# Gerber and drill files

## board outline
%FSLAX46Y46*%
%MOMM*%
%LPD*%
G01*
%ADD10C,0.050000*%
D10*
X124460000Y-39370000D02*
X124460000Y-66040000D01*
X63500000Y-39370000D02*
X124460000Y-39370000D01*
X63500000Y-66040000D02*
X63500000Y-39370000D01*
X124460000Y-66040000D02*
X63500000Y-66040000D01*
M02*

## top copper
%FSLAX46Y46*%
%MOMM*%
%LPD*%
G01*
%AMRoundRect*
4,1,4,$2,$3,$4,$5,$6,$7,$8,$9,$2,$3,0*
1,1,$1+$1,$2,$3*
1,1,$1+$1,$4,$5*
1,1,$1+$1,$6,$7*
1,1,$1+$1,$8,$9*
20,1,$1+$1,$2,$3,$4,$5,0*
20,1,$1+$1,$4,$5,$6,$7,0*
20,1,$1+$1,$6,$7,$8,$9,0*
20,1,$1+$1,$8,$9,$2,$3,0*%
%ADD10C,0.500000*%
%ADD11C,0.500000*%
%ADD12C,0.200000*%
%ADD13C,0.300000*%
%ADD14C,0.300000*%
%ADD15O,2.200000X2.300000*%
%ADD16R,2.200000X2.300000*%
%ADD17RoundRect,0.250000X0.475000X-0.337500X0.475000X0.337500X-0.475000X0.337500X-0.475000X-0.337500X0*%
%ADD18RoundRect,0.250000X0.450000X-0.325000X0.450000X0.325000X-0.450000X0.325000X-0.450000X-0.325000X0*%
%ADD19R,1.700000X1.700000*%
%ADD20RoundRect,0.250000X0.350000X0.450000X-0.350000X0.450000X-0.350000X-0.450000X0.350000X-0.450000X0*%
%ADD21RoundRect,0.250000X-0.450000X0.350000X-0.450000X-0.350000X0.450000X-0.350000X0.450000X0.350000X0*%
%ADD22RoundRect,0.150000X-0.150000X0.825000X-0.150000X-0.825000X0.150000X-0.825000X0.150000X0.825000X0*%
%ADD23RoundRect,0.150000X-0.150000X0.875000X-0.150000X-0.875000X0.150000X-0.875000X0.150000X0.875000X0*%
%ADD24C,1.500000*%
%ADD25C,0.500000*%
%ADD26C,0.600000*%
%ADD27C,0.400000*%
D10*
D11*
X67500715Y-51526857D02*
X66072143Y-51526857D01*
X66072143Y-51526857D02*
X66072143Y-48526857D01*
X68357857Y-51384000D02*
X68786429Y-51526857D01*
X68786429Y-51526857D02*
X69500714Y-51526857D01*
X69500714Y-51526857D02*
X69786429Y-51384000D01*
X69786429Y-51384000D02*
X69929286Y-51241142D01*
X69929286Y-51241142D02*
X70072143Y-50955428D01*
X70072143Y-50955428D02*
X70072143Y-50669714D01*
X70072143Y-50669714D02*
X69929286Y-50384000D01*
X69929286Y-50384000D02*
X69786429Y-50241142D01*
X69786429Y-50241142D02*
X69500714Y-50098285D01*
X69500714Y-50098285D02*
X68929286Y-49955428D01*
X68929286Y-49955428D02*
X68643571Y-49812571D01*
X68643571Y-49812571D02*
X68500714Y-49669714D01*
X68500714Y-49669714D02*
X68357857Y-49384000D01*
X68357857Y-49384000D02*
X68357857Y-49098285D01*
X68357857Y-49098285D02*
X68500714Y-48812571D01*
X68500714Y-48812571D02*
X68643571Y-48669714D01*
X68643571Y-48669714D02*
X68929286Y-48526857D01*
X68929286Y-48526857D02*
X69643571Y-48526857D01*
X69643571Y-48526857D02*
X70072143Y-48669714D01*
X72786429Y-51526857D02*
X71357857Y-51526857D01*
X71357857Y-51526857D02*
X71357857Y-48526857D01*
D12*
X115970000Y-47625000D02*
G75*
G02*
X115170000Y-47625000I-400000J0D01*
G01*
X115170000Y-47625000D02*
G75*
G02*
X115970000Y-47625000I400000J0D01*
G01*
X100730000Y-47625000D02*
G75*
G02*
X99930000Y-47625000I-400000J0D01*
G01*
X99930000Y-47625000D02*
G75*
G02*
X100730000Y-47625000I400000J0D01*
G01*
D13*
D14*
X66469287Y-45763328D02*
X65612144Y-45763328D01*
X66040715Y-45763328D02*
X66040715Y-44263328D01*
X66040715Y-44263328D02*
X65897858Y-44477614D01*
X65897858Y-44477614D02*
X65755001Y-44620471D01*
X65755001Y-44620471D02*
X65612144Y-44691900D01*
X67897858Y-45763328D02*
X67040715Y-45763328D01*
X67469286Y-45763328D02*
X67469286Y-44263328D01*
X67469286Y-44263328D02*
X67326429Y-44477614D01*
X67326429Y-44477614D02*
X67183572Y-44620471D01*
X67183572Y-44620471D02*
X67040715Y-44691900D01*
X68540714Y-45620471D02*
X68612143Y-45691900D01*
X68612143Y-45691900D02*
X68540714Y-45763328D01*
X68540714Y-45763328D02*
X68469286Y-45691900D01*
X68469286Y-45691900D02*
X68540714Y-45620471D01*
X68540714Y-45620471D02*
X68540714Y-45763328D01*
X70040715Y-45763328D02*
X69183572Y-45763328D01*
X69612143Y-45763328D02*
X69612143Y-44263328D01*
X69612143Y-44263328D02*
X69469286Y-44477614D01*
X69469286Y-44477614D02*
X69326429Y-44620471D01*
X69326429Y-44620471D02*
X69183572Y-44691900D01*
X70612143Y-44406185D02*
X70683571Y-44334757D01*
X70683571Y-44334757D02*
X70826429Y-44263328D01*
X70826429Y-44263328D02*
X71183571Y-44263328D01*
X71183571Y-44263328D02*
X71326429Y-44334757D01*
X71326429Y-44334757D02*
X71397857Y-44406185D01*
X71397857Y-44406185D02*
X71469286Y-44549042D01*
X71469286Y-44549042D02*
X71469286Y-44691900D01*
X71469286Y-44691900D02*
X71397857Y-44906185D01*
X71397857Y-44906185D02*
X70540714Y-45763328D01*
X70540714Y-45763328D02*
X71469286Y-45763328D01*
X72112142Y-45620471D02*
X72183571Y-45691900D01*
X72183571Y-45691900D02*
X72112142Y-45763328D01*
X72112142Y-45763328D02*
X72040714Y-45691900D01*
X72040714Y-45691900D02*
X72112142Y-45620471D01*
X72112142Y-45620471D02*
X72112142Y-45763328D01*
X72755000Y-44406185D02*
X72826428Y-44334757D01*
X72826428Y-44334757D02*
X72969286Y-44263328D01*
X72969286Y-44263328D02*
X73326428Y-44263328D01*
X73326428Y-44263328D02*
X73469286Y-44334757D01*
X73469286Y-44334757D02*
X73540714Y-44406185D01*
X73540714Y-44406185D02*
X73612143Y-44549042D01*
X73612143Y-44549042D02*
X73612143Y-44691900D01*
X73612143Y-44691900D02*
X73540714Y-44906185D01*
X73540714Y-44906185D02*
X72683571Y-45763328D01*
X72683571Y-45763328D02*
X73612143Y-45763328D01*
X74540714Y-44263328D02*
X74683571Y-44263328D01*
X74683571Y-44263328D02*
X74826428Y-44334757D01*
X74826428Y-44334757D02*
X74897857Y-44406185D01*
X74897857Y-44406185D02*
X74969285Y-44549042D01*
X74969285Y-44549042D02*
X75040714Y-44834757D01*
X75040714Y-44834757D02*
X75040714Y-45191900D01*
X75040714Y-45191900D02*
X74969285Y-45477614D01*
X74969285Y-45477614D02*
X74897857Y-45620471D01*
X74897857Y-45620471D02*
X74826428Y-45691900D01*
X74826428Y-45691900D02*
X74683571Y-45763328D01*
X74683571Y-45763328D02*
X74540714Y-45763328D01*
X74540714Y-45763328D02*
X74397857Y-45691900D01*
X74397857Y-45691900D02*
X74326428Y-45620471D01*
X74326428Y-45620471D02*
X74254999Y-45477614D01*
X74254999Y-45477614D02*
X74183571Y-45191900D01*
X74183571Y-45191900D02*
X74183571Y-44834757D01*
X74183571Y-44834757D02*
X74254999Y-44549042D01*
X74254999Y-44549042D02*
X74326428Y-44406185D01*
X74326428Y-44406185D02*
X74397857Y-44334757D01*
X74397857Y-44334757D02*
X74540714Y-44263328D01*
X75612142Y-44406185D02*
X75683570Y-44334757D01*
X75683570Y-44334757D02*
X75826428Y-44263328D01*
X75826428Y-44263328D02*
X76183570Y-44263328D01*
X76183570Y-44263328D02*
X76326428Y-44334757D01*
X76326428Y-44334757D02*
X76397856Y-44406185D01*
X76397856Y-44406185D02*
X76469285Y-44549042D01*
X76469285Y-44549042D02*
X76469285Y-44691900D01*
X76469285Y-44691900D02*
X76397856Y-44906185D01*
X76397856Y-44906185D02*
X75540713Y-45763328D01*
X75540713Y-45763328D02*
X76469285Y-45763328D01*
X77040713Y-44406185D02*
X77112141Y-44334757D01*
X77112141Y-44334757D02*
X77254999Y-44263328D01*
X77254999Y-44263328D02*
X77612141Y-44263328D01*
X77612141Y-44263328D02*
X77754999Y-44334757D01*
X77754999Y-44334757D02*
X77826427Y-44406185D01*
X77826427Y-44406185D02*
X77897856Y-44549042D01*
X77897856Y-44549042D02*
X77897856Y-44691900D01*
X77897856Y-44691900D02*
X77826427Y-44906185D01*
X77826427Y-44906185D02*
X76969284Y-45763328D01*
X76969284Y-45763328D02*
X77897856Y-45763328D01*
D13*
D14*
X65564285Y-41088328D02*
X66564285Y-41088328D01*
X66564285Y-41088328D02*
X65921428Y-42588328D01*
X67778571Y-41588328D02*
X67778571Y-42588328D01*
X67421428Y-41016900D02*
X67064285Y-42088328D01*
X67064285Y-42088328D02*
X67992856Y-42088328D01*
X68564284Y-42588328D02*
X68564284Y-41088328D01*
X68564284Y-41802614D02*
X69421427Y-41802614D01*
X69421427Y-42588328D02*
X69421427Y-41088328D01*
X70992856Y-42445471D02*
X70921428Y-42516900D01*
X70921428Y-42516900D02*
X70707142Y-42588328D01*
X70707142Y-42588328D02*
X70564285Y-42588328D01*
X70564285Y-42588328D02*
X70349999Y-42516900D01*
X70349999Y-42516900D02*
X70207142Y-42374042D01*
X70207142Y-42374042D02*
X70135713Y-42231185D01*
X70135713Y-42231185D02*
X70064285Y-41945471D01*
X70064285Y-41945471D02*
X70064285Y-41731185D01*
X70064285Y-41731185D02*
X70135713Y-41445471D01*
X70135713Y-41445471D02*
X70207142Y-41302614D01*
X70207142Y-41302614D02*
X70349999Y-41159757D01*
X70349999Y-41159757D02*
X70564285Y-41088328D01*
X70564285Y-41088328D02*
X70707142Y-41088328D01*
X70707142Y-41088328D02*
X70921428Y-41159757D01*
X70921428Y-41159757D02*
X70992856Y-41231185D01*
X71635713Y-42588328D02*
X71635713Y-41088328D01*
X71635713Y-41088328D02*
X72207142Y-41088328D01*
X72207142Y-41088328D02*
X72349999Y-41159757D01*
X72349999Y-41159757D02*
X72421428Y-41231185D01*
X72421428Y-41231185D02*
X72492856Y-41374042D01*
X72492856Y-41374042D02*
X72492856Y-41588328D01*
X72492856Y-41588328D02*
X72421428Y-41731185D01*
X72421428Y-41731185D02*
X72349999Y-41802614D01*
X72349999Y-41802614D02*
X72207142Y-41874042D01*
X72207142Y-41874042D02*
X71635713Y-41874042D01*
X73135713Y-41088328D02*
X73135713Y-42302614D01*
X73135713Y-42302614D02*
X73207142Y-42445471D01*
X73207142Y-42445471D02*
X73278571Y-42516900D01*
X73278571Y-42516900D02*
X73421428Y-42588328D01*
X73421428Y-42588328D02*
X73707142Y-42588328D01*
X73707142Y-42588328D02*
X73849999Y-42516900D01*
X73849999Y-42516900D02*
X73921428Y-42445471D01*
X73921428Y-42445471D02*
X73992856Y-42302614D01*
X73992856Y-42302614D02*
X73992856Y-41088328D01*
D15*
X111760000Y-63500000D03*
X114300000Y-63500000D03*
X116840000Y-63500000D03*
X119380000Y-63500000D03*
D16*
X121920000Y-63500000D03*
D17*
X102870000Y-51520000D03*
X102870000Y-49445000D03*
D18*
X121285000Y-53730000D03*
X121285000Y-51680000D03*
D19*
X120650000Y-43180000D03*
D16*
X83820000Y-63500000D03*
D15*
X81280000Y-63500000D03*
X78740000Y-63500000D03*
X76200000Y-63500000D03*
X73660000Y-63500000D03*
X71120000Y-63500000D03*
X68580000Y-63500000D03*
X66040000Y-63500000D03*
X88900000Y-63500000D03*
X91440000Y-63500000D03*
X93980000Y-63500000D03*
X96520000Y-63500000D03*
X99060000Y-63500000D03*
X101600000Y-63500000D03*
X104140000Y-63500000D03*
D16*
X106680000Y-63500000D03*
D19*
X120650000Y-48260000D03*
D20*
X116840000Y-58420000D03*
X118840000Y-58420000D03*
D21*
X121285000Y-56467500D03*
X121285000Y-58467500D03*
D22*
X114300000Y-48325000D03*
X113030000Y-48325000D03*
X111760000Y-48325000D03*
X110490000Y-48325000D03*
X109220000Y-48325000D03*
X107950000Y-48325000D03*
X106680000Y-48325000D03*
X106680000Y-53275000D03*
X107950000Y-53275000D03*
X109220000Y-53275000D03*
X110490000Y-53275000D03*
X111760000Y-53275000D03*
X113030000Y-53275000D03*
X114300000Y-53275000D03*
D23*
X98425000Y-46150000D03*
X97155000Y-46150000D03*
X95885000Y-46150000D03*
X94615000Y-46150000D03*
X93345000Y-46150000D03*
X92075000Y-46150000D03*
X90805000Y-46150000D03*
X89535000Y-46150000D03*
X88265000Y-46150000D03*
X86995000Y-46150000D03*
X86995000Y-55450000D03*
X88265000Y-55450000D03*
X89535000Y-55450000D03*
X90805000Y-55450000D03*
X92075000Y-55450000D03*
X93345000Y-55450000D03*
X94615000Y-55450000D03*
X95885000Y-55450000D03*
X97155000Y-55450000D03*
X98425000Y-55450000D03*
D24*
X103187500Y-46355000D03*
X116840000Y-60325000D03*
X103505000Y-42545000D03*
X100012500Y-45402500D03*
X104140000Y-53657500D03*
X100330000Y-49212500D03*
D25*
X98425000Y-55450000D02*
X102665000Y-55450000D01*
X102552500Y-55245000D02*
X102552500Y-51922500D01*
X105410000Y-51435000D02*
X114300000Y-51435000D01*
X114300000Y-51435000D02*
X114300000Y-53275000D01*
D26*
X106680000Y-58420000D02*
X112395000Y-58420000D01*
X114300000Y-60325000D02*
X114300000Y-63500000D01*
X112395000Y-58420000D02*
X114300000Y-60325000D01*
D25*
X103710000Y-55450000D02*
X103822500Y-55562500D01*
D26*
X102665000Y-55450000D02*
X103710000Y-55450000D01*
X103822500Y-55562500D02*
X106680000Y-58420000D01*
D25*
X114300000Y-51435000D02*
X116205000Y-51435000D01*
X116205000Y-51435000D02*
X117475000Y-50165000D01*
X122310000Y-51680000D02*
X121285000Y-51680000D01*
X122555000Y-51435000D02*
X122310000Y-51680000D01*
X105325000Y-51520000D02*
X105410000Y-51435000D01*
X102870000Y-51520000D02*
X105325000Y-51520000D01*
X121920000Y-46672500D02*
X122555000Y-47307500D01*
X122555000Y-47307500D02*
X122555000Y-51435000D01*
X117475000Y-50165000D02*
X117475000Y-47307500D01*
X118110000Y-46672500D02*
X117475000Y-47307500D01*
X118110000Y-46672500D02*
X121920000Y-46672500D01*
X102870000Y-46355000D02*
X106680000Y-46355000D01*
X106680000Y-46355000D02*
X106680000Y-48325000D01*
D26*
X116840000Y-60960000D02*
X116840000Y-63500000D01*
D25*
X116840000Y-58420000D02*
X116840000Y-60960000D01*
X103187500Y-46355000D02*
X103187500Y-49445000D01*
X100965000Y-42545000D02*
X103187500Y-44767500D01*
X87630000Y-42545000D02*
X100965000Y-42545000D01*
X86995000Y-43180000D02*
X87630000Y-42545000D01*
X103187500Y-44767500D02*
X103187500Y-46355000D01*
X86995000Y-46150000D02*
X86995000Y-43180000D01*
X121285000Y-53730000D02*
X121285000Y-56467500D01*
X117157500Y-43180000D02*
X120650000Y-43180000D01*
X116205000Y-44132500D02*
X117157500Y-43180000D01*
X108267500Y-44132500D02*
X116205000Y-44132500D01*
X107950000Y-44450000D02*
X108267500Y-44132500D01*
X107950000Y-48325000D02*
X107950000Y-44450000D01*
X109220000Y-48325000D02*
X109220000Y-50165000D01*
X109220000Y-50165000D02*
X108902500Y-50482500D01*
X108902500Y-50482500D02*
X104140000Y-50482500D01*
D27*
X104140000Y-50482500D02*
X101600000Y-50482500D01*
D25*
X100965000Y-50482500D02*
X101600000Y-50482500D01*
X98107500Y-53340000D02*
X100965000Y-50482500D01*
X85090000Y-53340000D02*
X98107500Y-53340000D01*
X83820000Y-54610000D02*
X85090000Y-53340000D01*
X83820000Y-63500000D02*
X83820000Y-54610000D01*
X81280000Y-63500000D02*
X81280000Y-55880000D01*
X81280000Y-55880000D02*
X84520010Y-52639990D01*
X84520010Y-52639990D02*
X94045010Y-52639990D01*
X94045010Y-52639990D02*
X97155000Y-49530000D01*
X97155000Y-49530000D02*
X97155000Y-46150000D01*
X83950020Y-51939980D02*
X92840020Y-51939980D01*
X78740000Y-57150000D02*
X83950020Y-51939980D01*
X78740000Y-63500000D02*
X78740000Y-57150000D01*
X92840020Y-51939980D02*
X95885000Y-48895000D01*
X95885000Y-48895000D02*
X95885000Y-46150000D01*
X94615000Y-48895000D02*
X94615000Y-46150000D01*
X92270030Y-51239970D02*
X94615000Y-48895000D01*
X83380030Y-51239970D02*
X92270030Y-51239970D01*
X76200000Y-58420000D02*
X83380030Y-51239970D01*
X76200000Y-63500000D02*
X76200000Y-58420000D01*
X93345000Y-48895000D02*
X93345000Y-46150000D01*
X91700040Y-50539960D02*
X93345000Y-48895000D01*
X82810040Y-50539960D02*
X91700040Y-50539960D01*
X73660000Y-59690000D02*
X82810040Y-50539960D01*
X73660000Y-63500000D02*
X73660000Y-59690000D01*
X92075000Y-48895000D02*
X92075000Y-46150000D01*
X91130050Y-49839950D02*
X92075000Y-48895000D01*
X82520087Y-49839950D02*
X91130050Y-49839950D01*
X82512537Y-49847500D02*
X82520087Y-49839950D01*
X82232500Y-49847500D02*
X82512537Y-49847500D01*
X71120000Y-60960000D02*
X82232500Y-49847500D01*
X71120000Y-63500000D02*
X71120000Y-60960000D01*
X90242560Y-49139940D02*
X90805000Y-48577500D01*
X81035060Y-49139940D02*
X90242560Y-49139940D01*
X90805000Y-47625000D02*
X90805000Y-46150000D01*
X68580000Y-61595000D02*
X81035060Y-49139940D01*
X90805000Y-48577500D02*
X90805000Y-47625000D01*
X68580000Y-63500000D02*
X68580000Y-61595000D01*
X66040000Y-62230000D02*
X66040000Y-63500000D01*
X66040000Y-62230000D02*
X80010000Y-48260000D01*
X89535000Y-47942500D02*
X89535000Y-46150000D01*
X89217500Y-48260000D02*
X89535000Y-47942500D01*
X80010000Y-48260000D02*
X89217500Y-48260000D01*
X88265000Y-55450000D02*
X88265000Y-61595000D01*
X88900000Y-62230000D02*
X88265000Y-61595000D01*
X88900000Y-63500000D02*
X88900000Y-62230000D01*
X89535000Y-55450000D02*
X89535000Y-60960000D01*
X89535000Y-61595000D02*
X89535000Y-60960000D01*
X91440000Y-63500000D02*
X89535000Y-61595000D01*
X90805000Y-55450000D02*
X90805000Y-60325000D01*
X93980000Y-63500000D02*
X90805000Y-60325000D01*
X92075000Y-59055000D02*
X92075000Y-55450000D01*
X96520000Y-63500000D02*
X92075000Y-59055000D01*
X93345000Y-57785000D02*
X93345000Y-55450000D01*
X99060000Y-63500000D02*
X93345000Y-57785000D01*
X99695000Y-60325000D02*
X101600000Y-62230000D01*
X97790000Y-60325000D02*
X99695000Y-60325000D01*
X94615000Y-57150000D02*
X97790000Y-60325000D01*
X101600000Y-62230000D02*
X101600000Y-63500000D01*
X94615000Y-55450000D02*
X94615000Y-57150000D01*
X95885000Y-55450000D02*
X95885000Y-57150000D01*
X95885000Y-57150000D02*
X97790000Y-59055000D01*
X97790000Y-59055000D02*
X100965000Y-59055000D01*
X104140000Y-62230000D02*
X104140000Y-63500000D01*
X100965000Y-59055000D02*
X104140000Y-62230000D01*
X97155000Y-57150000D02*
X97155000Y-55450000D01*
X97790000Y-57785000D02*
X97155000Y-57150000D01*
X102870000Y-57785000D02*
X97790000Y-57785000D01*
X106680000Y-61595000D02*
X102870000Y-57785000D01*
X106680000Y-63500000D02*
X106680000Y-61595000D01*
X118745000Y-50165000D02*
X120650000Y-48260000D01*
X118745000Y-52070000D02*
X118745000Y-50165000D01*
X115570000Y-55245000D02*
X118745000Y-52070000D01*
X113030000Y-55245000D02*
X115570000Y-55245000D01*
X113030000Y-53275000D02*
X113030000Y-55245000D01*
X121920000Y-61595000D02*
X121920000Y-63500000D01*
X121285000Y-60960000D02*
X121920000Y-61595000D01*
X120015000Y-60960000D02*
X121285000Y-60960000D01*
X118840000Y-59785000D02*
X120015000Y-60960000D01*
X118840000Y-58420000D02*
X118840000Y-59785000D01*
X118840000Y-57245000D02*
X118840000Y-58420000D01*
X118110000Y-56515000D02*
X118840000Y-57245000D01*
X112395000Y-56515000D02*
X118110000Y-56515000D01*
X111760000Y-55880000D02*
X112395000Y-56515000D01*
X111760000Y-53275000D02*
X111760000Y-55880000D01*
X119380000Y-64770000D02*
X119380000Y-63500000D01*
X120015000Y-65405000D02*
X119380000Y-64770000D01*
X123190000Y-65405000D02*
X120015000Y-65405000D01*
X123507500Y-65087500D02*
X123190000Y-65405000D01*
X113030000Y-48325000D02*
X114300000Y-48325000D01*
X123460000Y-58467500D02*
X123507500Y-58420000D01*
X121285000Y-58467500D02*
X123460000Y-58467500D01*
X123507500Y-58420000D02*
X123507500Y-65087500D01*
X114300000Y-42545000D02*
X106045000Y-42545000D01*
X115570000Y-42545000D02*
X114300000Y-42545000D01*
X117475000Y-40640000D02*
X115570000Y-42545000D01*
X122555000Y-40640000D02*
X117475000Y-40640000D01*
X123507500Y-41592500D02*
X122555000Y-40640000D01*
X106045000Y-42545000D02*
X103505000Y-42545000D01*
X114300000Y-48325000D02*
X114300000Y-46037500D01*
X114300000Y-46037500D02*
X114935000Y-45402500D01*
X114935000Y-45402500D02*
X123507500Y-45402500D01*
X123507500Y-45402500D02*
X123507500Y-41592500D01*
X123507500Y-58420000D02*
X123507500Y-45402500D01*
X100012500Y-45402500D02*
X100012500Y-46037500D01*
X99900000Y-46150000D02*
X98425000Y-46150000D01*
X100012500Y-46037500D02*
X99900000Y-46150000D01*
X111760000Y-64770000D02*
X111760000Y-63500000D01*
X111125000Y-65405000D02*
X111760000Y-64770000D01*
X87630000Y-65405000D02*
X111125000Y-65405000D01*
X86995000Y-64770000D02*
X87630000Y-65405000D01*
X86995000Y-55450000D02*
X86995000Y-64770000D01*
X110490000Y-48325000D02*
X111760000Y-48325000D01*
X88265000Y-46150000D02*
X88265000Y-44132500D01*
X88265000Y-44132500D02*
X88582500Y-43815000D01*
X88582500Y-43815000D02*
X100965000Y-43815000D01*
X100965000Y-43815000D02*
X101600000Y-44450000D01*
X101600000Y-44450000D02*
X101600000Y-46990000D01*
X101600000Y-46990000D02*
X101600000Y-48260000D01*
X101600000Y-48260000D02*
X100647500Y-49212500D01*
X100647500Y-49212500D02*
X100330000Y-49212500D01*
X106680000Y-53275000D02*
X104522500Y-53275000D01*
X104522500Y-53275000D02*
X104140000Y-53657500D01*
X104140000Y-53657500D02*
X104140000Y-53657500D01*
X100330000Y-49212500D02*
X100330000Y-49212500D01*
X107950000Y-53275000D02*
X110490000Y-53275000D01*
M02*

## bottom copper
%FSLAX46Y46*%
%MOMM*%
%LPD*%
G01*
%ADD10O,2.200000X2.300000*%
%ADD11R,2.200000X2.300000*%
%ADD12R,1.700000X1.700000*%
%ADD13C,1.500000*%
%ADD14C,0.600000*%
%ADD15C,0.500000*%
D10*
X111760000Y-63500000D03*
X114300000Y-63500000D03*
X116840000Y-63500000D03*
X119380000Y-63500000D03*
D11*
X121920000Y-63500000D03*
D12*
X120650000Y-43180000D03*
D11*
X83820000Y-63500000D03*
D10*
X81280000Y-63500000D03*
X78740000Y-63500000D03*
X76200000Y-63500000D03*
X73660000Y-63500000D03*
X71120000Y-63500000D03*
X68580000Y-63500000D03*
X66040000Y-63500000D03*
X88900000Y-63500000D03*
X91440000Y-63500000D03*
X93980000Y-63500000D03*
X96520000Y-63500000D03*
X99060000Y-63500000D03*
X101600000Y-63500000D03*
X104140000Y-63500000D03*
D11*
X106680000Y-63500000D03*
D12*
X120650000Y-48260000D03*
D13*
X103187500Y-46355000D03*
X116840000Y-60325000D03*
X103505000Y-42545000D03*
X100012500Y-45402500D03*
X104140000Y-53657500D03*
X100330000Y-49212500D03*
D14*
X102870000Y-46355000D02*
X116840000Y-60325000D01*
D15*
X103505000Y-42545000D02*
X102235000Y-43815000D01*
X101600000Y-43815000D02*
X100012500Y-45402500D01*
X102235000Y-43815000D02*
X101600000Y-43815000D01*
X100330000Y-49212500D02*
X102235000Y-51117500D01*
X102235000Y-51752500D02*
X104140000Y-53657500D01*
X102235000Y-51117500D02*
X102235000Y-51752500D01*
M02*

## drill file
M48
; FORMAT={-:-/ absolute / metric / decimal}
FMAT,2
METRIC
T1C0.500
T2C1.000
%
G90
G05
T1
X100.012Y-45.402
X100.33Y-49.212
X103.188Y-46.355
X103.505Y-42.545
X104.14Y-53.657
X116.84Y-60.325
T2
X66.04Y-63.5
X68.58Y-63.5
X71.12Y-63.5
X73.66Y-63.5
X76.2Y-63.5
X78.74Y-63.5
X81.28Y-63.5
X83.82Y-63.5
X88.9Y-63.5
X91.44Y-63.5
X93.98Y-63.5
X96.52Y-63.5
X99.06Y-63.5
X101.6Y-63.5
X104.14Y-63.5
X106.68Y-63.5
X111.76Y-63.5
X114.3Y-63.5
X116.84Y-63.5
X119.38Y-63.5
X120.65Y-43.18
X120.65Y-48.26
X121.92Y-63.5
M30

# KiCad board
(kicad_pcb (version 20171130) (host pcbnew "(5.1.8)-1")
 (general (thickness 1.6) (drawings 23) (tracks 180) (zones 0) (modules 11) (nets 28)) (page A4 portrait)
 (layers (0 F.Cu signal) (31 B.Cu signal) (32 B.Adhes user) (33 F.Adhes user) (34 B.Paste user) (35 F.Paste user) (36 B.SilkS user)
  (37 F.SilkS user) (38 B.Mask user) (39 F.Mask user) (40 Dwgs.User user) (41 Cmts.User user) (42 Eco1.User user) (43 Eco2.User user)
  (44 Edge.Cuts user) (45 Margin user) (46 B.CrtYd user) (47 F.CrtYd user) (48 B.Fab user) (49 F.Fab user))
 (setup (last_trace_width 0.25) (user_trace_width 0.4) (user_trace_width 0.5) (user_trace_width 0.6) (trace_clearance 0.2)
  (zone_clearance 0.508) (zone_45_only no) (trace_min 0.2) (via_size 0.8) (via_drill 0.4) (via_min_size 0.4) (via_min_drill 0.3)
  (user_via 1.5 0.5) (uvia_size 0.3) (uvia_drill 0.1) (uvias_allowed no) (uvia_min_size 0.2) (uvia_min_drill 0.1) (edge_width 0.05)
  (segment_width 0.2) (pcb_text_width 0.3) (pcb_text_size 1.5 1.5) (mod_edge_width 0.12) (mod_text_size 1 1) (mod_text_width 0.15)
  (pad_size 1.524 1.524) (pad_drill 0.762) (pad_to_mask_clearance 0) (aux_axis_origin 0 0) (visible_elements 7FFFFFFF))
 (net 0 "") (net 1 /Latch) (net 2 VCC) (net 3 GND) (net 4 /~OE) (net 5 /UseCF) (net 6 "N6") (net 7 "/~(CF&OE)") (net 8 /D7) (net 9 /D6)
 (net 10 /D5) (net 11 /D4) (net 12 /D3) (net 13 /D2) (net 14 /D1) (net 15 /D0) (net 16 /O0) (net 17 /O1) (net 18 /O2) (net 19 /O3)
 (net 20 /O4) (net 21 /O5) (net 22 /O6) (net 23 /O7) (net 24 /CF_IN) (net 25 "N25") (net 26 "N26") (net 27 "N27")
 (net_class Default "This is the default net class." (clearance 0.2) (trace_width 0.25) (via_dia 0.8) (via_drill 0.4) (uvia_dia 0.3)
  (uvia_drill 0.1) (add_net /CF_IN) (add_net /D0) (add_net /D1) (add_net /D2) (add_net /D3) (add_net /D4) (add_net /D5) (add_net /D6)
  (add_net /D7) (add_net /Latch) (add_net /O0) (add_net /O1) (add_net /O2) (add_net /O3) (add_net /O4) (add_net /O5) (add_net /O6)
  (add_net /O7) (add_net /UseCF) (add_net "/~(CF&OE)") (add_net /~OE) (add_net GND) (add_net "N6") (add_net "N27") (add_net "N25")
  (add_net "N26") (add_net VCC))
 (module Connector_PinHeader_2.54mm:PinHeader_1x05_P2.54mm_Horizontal (layer F.Cu) (at 121.92 63.5 270)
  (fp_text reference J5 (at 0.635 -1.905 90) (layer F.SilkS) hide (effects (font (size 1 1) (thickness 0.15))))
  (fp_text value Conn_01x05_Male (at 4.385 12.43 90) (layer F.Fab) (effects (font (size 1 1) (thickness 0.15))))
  (pad 5 thru_hole oval (at 0 10.16 270) (size 2.3 2.2) (drill 1) (layers *.Cu *.Mask) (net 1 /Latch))
  (pad 4 thru_hole oval (at 0 7.62 270) (size 2.3 2.2) (drill 1) (layers *.Cu *.Mask) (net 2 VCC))
  (pad 3 thru_hole oval (at 0 5.08 270) (size 2.3 2.2) (drill 1) (layers *.Cu *.Mask) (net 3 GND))
  (pad 2 thru_hole oval (at 0 2.54 270) (size 2.3 2.2) (drill 1) (layers *.Cu *.Mask) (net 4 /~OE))
  (pad 1 thru_hole rect (at 0 0 270) (size 2.3 2.2) (drill 1) (layers *.Cu *.Mask) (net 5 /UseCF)))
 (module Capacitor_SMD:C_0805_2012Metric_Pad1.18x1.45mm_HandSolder (layer F.Cu) (at 102.87 50.4825 90)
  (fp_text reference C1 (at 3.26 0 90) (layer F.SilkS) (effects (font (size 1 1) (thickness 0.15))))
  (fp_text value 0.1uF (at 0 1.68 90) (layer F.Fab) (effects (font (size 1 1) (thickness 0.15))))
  (pad 1 smd roundrect (at -1.0375 0 90) (size 1.175 1.45) (layers F.Cu F.Paste F.Mask) (roundrect_rratio 0.212766) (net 2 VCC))
  (pad 2 smd roundrect (at 1.0375 0 90) (size 1.175 1.45) (layers F.Cu F.Paste F.Mask) (roundrect_rratio 0.212766) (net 3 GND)))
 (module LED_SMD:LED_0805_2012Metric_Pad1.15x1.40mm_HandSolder (layer F.Cu) (at 121.285 52.705 90)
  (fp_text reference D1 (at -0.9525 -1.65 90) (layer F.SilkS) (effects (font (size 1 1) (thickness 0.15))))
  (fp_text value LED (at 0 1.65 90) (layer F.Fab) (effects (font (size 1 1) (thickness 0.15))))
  (pad 1 smd roundrect (at -1.025 0 90) (size 1.15 1.4) (layers F.Cu F.Paste F.Mask) (roundrect_rratio 0.217391) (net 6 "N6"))
  (pad 2 smd roundrect (at 1.025 0 90) (size 1.15 1.4) (layers F.Cu F.Paste F.Mask) (roundrect_rratio 0.217391) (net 2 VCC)))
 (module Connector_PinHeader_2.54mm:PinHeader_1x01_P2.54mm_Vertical (layer F.Cu) (at 120.65 43.18)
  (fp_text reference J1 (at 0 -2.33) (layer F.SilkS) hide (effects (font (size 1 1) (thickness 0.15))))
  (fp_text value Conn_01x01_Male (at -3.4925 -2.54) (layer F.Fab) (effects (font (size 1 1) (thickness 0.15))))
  (pad 1 thru_hole rect (at 0 0) (size 1.7 1.7) (drill 1) (layers *.Cu *.Mask) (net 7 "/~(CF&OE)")))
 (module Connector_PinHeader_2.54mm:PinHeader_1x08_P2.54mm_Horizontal (layer F.Cu) (at 83.82 63.5 270)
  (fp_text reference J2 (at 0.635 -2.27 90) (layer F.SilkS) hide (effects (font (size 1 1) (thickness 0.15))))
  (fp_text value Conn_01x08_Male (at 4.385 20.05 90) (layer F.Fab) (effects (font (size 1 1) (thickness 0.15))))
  (pad 1 thru_hole rect (at 0 0 270) (size 2.3 2.2) (drill 1) (layers *.Cu *.Mask) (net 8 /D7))
  (pad 2 thru_hole oval (at 0 2.54 270) (size 2.3 2.2) (drill 1) (layers *.Cu *.Mask) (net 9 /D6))
  (pad 3 thru_hole oval (at 0 5.08 270) (size 2.3 2.2) (drill 1) (layers *.Cu *.Mask) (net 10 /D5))
  (pad 4 thru_hole oval (at 0 7.62 270) (size 2.3 2.2) (drill 1) (layers *.Cu *.Mask) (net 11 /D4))
  (pad 5 thru_hole oval (at 0 10.16 270) (size 2.3 2.2) (drill 1) (layers *.Cu *.Mask) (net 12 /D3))
  (pad 6 thru_hole oval (at 0 12.7 270) (size 2.3 2.2) (drill 1) (layers *.Cu *.Mask) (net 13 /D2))
  (pad 7 thru_hole oval (at 0 15.24 270) (size 2.3 2.2) (drill 1) (layers *.Cu *.Mask) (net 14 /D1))
  (pad 8 thru_hole oval (at 0 17.78 270) (size 2.3 2.2) (drill 1) (layers *.Cu *.Mask) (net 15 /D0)))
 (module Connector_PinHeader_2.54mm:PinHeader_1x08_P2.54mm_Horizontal (layer F.Cu) (at 106.68 63.5 270)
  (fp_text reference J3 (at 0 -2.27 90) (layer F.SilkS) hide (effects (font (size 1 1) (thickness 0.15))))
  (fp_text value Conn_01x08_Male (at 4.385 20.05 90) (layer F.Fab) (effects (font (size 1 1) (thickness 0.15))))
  (pad 8 thru_hole oval (at 0 17.78 270) (size 2.3 2.2) (drill 1) (layers *.Cu *.Mask) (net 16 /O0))
  (pad 7 thru_hole oval (at 0 15.24 270) (size 2.3 2.2) (drill 1) (layers *.Cu *.Mask) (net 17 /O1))
  (pad 6 thru_hole oval (at 0 12.7 270) (size 2.3 2.2) (drill 1) (layers *.Cu *.Mask) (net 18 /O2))
  (pad 5 thru_hole oval (at 0 10.16 270) (size 2.3 2.2) (drill 1) (layers *.Cu *.Mask) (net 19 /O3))
  (pad 4 thru_hole oval (at 0 7.62 270) (size 2.3 2.2) (drill 1) (layers *.Cu *.Mask) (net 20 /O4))
  (pad 3 thru_hole oval (at 0 5.08 270) (size 2.3 2.2) (drill 1) (layers *.Cu *.Mask) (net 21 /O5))
  (pad 2 thru_hole oval (at 0 2.54 270) (size 2.3 2.2) (drill 1) (layers *.Cu *.Mask) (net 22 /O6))
  (pad 1 thru_hole rect (at 0 0 270) (size 2.3 2.2) (drill 1) (layers *.Cu *.Mask) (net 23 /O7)))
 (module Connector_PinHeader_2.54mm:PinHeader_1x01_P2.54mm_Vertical (layer F.Cu) (at 120.65 48.26)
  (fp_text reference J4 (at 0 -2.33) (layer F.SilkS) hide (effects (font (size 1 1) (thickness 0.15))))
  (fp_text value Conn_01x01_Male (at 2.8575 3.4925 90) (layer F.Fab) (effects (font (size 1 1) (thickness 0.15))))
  (pad 1 thru_hole rect (at 0 0) (size 1.7 1.7) (drill 1) (layers *.Cu *.Mask) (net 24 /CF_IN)))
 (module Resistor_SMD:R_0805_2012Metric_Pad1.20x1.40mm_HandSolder (layer F.Cu) (at 117.84 58.42 180)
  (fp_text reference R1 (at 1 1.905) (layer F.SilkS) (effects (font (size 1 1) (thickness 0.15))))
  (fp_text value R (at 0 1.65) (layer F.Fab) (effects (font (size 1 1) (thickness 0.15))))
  (pad 2 smd roundrect (at 1 0 180) (size 1.2 1.4) (layers F.Cu F.Paste F.Mask) (roundrect_rratio 0.208333) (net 3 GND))
  (pad 1 smd roundrect (at -1 0 180) (size 1.2 1.4) (layers F.Cu F.Paste F.Mask) (roundrect_rratio 0.208333) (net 5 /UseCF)))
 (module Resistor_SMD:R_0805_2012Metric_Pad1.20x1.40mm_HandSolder (layer F.Cu) (at 121.285 57.4675 270)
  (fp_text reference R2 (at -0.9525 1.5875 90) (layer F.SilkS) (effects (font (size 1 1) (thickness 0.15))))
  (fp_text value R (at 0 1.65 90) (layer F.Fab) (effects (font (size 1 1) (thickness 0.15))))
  (pad 1 smd roundrect (at -1 0 270) (size 1.2 1.4) (layers F.Cu F.Paste F.Mask) (roundrect_rratio 0.208333) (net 6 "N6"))
  (pad 2 smd roundrect (at 1 0 270) (size 1.2 1.4) (layers F.Cu F.Paste F.Mask) (roundrect_rratio 0.208333) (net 4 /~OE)))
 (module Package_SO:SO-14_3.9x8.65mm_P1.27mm (layer F.Cu) (at 110.49 50.8 270)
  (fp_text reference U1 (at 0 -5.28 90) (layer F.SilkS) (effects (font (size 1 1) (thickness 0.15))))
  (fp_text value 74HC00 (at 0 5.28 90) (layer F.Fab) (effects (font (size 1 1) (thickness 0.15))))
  (pad 1 smd roundrect (at -2.475 -3.81 270) (size 1.95 0.6) (layers F.Cu F.Paste F.Mask) (roundrect_rratio 0.25) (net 4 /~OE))
  (pad 2 smd roundrect (at -2.475 -2.54 270) (size 1.95 0.6) (layers F.Cu F.Paste F.Mask) (roundrect_rratio 0.25) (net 4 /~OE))
  (pad 3 smd roundrect (at -2.475 -1.27 270) (size 1.95 0.6) (layers F.Cu F.Paste F.Mask) (roundrect_rratio 0.25) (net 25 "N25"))
  (pad 4 smd roundrect (at -2.475 0 270) (size 1.95 0.6) (layers F.Cu F.Paste F.Mask) (roundrect_rratio 0.25) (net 25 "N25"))
  (pad 5 smd roundrect (at -2.475 1.27 270) (size 1.95 0.6) (layers F.Cu F.Paste F.Mask) (roundrect_rratio 0.25) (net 8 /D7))
  (pad 6 smd roundrect (at -2.475 2.54 270) (size 1.95 0.6) (layers F.Cu F.Paste F.Mask) (roundrect_rratio 0.25) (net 7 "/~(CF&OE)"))
  (pad 7 smd roundrect (at -2.475 3.81 270) (size 1.95 0.6) (layers F.Cu F.Paste F.Mask) (roundrect_rratio 0.25) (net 3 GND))
  (pad 8 smd roundrect (at 2.475 3.81 270) (size 1.95 0.6) (layers F.Cu F.Paste F.Mask) (roundrect_rratio 0.25) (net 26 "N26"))
  (pad 9 smd roundrect (at 2.475 2.54 270) (size 1.95 0.6) (layers F.Cu F.Paste F.Mask) (roundrect_rratio 0.25) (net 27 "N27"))
  (pad 10 smd roundrect (at 2.475 1.27 270) (size 1.95 0.6) (layers F.Cu F.Paste F.Mask) (roundrect_rratio 0.25) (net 27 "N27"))
  (pad 11 smd roundrect (at 2.475 0 270) (size 1.95 0.6) (layers F.Cu F.Paste F.Mask) (roundrect_rratio 0.25) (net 27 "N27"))
  (pad 12 smd roundrect (at 2.475 -1.27 270) (size 1.95 0.6) (layers F.Cu F.Paste F.Mask) (roundrect_rratio 0.25) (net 5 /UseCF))
  (pad 13 smd roundrect (at 2.475 -2.54 270) (size 1.95 0.6) (layers F.Cu F.Paste F.Mask) (roundrect_rratio 0.25) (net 24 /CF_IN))
  (pad 14 smd roundrect (at 2.475 -3.81 270) (size 1.95 0.6) (layers F.Cu F.Paste F.Mask) (roundrect_rratio 0.25) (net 2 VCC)))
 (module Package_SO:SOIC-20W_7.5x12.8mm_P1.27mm (layer F.Cu) (at 92.71 50.8 270)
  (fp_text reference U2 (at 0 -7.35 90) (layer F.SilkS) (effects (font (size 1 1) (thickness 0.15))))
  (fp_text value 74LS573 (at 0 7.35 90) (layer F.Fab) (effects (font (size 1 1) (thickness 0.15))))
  (pad 1 smd roundrect (at -4.65 -5.715 270) (size 2.05 0.6) (layers F.Cu F.Paste F.Mask) (roundrect_rratio 0.25) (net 4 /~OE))
  (pad 2 smd roundrect (at -4.65 -4.445 270) (size 2.05 0.6) (layers F.Cu F.Paste F.Mask) (roundrect_rratio 0.25) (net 9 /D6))
  (pad 3 smd roundrect (at -4.65 -3.175 270) (size 2.05 0.6) (layers F.Cu F.Paste F.Mask) (roundrect_rratio 0.25) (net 10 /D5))
  (pad 4 smd roundrect (at -4.65 -1.905 270) (size 2.05 0.6) (layers F.Cu F.Paste F.Mask) (roundrect_rratio 0.25) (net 11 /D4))
  (pad 5 smd roundrect (at -4.65 -0.635 270) (size 2.05 0.6) (layers F.Cu F.Paste F.Mask) (roundrect_rratio 0.25) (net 12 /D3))
  (pad 6 smd roundrect (at -4.65 0.635 270) (size 2.05 0.6) (layers F.Cu F.Paste F.Mask) (roundrect_rratio 0.25) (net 13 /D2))
  (pad 7 smd roundrect (at -4.65 1.905 270) (size 2.05 0.6) (layers F.Cu F.Paste F.Mask) (roundrect_rratio 0.25) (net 14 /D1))
  (pad 8 smd roundrect (at -4.65 3.175 270) (size 2.05 0.6) (layers F.Cu F.Paste F.Mask) (roundrect_rratio 0.25) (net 15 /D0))
  (pad 9 smd roundrect (at -4.65 4.445 270) (size 2.05 0.6) (layers F.Cu F.Paste F.Mask) (roundrect_rratio 0.25) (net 26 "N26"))
  (pad 10 smd roundrect (at -4.65 5.715 270) (size 2.05 0.6) (layers F.Cu F.Paste F.Mask) (roundrect_rratio 0.25) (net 3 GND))
  (pad 11 smd roundrect (at 4.65 5.715 270) (size 2.05 0.6) (layers F.Cu F.Paste F.Mask) (roundrect_rratio 0.25) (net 1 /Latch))
  (pad 12 smd roundrect (at 4.65 4.445 270) (size 2.05 0.6) (layers F.Cu F.Paste F.Mask) (roundrect_rratio 0.25) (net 16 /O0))
  (pad 13 smd roundrect (at 4.65 3.175 270) (size 2.05 0.6) (layers F.Cu F.Paste F.Mask) (roundrect_rratio 0.25) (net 17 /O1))
  (pad 14 smd roundrect (at 4.65 1.905 270) (size 2.05 0.6) (layers F.Cu F.Paste F.Mask) (roundrect_rratio 0.25) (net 18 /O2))
  (pad 15 smd roundrect (at 4.65 0.635 270) (size 2.05 0.6) (layers F.Cu F.Paste F.Mask) (roundrect_rratio 0.25) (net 19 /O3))
  (pad 16 smd roundrect (at 4.65 -0.635 270) (size 2.05 0.6) (layers F.Cu F.Paste F.Mask) (roundrect_rratio 0.25) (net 20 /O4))
  (pad 17 smd roundrect (at 4.65 -1.905 270) (size 2.05 0.6) (layers F.Cu F.Paste F.Mask) (roundrect_rratio 0.25) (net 21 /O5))
  (pad 18 smd roundrect (at 4.65 -3.175 270) (size 2.05 0.6) (layers F.Cu F.Paste F.Mask) (roundrect_rratio 0.25) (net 22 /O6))
  (pad 19 smd roundrect (at 4.65 -4.445 270) (size 2.05 0.6) (layers F.Cu F.Paste F.Mask) (roundrect_rratio 0.25) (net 23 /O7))
  (pad 20 smd roundrect (at 4.65 -5.715 270) (size 2.05 0.6) (layers F.Cu F.Paste F.Mask) (roundrect_rratio 0.25) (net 2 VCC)))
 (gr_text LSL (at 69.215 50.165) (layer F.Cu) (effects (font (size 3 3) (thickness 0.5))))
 (gr_circle (center 115.57 47.625) (end 115.97 47.625) (layer F.Cu) (width 0.2))
 (gr_circle (center 100.33 47.625) (end 100.73 47.625) (layer F.Cu) (width 0.2))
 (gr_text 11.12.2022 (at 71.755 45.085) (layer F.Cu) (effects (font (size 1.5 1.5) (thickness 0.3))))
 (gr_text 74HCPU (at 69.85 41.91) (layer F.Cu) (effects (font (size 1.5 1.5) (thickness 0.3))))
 (gr_line (start 124.46 39.37) (end 124.46 66.04) (layer Edge.Cuts) (width 0.05))
 (gr_line (start 63.5 39.37) (end 124.46 39.37) (layer Edge.Cuts) (width 0.05))
 (gr_line (start 63.5 66.04) (end 63.5 39.37) (layer Edge.Cuts) (width 0.05))
 (gr_line (start 124.46 66.04) (end 63.5 66.04) (layer Edge.Cuts) (width 0.05))
 (segment (start 98.425 55.45) (end 102.665 55.45) (width 0.5) (layer F.Cu) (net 2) (status 10))
 (segment (start 102.5525 55.245) (end 102.5525 51.9225) (width 0.5) (layer F.Cu) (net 2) (status 20))
 (segment (start 105.41 51.435) (end 114.3 51.435) (width 0.5) (layer F.Cu) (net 2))
 (segment (start 114.3 51.435) (end 114.3 53.275) (width 0.5) (layer F.Cu) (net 2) (status 20))
 (segment (start 106.68 58.42) (end 112.395 58.42) (width 0.6) (layer F.Cu) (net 2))
 (segment (start 114.3 60.325) (end 114.3 63.5) (width 0.6) (layer F.Cu) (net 2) (status 20))
 (segment (start 112.395 58.42) (end 114.3 60.325) (width 0.6) (layer F.Cu) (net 2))
 (segment (start 103.71 55.45) (end 103.8225 55.5625) (width 0.5) (layer F.Cu) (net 2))
 (segment (start 102.665 55.45) (end 103.71 55.45) (width 0.6) (layer F.Cu) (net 2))
 (segment (start 103.8225 55.5625) (end 106.68 58.42) (width 0.6) (layer F.Cu) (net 2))
 (segment (start 114.3 51.435) (end 116.205 51.435) (width 0.5) (layer F.Cu) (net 2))
 (segment (start 116.205 51.435) (end 117.475 50.165) (width 0.5) (layer F.Cu) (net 2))
 (segment (start 122.31 51.68) (end 121.285 51.68) (width 0.5) (layer F.Cu) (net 2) (status 20))
 (segment (start 122.555 51.435) (end 122.31 51.68) (width 0.5) (layer F.Cu) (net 2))
 (segment (start 105.325 51.52) (end 105.41 51.435) (width 0.5) (layer F.Cu) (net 2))
 (segment (start 102.87 51.52) (end 105.325 51.52) (width 0.5) (layer F.Cu) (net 2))
 (segment (start 121.92 46.6725) (end 122.555 47.3075) (width 0.5) (layer F.Cu) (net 2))
 (segment (start 122.555 47.3075) (end 122.555 51.435) (width 0.5) (layer F.Cu) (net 2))
 (segment (start 117.475 50.165) (end 117.475 47.3075) (width 0.5) (layer F.Cu) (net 2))
 (segment (start 118.11 46.6725) (end 117.475 47.3075) (width 0.5) (layer F.Cu) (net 2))
 (segment (start 118.11 46.6725) (end 121.92 46.6725) (width 0.5) (layer F.Cu) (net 2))
 (segment (start 102.87 46.355) (end 106.68 46.355) (width 0.5) (layer F.Cu) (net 3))
 (segment (start 106.68 46.355) (end 106.68 48.325) (width 0.5) (layer F.Cu) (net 3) (status 20))
 (segment (start 116.84 60.96) (end 116.84 63.5) (width 0.6) (layer F.Cu) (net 3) (status 20))
 (segment (start 116.84 58.42) (end 116.84 60.96) (width 0.5) (layer F.Cu) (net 3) (status 10))
 (segment (start 103.1875 46.355) (end 103.1875 49.445) (width 0.5) (layer F.Cu) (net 3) (status 20))
 (via (at 103.1875 46.355) (size 1.5) (drill 0.5) (layers F.Cu B.Cu) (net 3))
 (segment (start 102.87 46.355) (end 116.84 60.325) (width 0.6) (layer B.Cu) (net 3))
 (via (at 116.84 60.325) (size 1.5) (drill 0.5) (layers F.Cu B.Cu) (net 3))
 (segment (start 100.965 42.545) (end 103.1875 44.7675) (width 0.5) (layer F.Cu) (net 3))
 (segment (start 87.63 42.545) (end 100.965 42.545) (width 0.5) (layer F.Cu) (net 3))
 (segment (start 86.995 43.18) (end 87.63 42.545) (width 0.5) (layer F.Cu) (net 3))
 (segment (start 103.1875 44.7675) (end 103.1875 46.355) (width 0.5) (layer F.Cu) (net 3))
 (segment (start 86.995 46.15) (end 86.995 43.18) (width 0.5) (layer F.Cu) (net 3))
 (segment (start 121.285 53.73) (end 121.285 56.4675) (width 0.5) (layer F.Cu) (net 6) (status 30))
 (segment (start 117.1575 43.18) (end 120.65 43.18) (width 0.5) (layer F.Cu) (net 7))
 (segment (start 116.205 44.1325) (end 117.1575 43.18) (width 0.5) (layer F.Cu) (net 7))
 (segment (start 108.2675 44.1325) (end 116.205 44.1325) (width 0.5) (layer F.Cu) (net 7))
 (segment (start 107.95 44.45) (end 108.2675 44.1325) (width 0.5) (layer F.Cu) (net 7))
 (segment (start 107.95 48.325) (end 107.95 44.45) (width 0.5) (layer F.Cu) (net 7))
 (segment (start 109.22 48.325) (end 109.22 50.165) (width 0.5) (layer F.Cu) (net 8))
 (segment (start 109.22 50.165) (end 108.9025 50.4825) (width 0.5) (layer F.Cu) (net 8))
 (segment (start 108.9025 50.4825) (end 104.14 50.4825) (width 0.5) (layer F.Cu) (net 8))
 (segment (start 104.14 50.4825) (end 101.6 50.4825) (width 0.4) (layer F.Cu) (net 8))
 (segment (start 100.965 50.4825) (end 101.6 50.4825) (width 0.5) (layer F.Cu) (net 8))
 (segment (start 98.1075 53.34) (end 100.965 50.4825) (width 0.5) (layer F.Cu) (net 8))
 (segment (start 85.09 53.34) (end 98.1075 53.34) (width 0.5) (layer F.Cu) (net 8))
 (segment (start 83.82 54.61) (end 85.09 53.34) (width 0.5) (layer F.Cu) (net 8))
 (segment (start 83.82 63.5) (end 83.82 54.61) (width 0.5) (layer F.Cu) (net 8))
 (segment (start 81.28 63.5) (end 81.28 55.88) (width 0.5) (layer F.Cu) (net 9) (status 10))
 (segment (start 81.28 55.88) (end 84.52001 52.63999) (width 0.5) (layer F.Cu) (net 9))
 (segment (start 84.52001 52.63999) (end 94.04501 52.63999) (width 0.5) (layer F.Cu) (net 9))
 (segment (start 94.04501 52.63999) (end 97.155 49.53) (width 0.5) (layer F.Cu) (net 9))
 (segment (start 97.155 49.53) (end 97.155 46.15) (width 0.5) (layer F.Cu) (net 9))
 (segment (start 83.95002 51.93998) (end 92.84002 51.93998) (width 0.5) (layer F.Cu) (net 10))
 (segment (start 78.74 57.15) (end 83.95002 51.93998) (width 0.5) (layer F.Cu) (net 10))
 (segment (start 78.74 63.5) (end 78.74 57.15) (width 0.5) (layer F.Cu) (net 10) (status 10))
 (segment (start 92.84002 51.93998) (end 95.885 48.895) (width 0.5) (layer F.Cu) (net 10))
 (segment (start 95.885 48.895) (end 95.885 46.15) (width 0.5) (layer F.Cu) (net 10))
 (segment (start 94.615 48.895) (end 94.615 46.15) (width 0.5) (layer F.Cu) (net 11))
 (segment (start 92.27003 51.23997) (end 94.615 48.895) (width 0.5) (layer F.Cu) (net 11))
 (segment (start 83.38003 51.23997) (end 92.27003 51.23997) (width 0.5) (layer F.Cu) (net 11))
 (segment (start 76.2 58.42) (end 83.38003 51.23997) (width 0.5) (layer F.Cu) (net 11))
 (segment (start 76.2 63.5) (end 76.2 58.42) (width 0.5) (layer F.Cu) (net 11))
 (segment (start 93.345 48.895) (end 93.345 46.15) (width 0.5) (layer F.Cu) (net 12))
 (segment (start 91.70004 50.53996) (end 93.345 48.895) (width 0.5) (layer F.Cu) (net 12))
 (segment (start 82.81004 50.53996) (end 91.70004 50.53996) (width 0.5) (layer F.Cu) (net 12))
 (segment (start 73.66 59.69) (end 82.81004 50.53996) (width 0.5) (layer F.Cu) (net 12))
 (segment (start 73.66 63.5) (end 73.66 59.69) (width 0.5) (layer F.Cu) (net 12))
 (segment (start 92.075 48.895) (end 92.075 46.15) (width 0.5) (layer F.Cu) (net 13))
 (segment (start 91.13005 49.83995) (end 92.075 48.895) (width 0.5) (layer F.Cu) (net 13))
 (segment (start 82.520087 49.83995) (end 91.13005 49.83995) (width 0.5) (layer F.Cu) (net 13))
 (segment (start 82.512537 49.8475) (end 82.520087 49.83995) (width 0.5) (layer F.Cu) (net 13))
 (segment (start 82.2325 49.8475) (end 82.512537 49.8475) (width 0.5) (layer F.Cu) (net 13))
 (segment (start 71.12 60.96) (end 82.2325 49.8475) (width 0.5) (layer F.Cu) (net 13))
 (segment (start 71.12 63.5) (end 71.12 60.96) (width 0.5) (layer F.Cu) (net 13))
 (segment (start 90.24256 49.13994) (end 90.805 48.5775) (width 0.5) (layer F.Cu) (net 14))
 (segment (start 81.03506 49.13994) (end 90.24256 49.13994) (width 0.5) (layer F.Cu) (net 14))
 (segment (start 90.805 47.625) (end 90.805 46.15) (width 0.5) (layer F.Cu) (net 14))
 (segment (start 68.58 61.595) (end 81.03506 49.13994) (width 0.5) (layer F.Cu) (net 14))
 (segment (start 90.805 48.5775) (end 90.805 47.625) (width 0.5) (layer F.Cu) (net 14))
 (segment (start 68.58 63.5) (end 68.58 61.595) (width 0.5) (layer F.Cu) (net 14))
 (segment (start 66.04 62.23) (end 66.04 63.5) (width 0.5) (layer F.Cu) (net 15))
 (segment (start 66.04 62.23) (end 80.01 48.26) (width 0.5) (layer F.Cu) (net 15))
 (segment (start 89.535 47.9425) (end 89.535 46.15) (width 0.5) (layer F.Cu) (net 15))
 (segment (start 89.2175 48.26) (end 89.535 47.9425) (width 0.5) (layer F.Cu) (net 15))
 (segment (start 80.01 48.26) (end 89.2175 48.26) (width 0.5) (layer F.Cu) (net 15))
 (segment (start 88.265 55.45) (end 88.265 61.595) (width 0.5) (layer F.Cu) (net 16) (status 10))
 (segment (start 88.9 62.23) (end 88.265 61.595) (width 0.5) (layer F.Cu) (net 16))
 (segment (start 88.9 63.5) (end 88.9 62.23) (width 0.5) (layer F.Cu) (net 16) (status 10))
 (segment (start 89.535 55.45) (end 89.535 60.96) (width 0.5) (layer F.Cu) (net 17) (status 10))
 (segment (start 89.535 61.595) (end 89.535 60.96) (width 0.5) (layer F.Cu) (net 17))
 (segment (start 91.44 63.5) (end 89.535 61.595) (width 0.5) (layer F.Cu) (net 17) (status 10))
 (segment (start 90.805 55.45) (end 90.805 60.325) (width 0.5) (layer F.Cu) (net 18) (status 10))
 (segment (start 93.98 63.5) (end 90.805 60.325) (width 0.5) (layer F.Cu) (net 18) (status 10))
 (segment (start 92.075 59.055) (end 92.075 55.45) (width 0.5) (layer F.Cu) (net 19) (status 20))
 (segment (start 96.52 63.5) (end 92.075 59.055) (width 0.5) (layer F.Cu) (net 19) (status 10))
 (segment (start 93.345 57.785) (end 93.345 55.45) (width 0.5) (layer F.Cu) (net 20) (status 20))
 (segment (start 99.06 63.5) (end 93.345 57.785) (width 0.5) (layer F.Cu) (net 20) (status 10))
 (segment (start 99.695 60.325) (end 101.6 62.23) (width 0.5) (layer F.Cu) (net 21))
 (segment (start 97.79 60.325) (end 99.695 60.325) (width 0.5) (layer F.Cu) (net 21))
 (segment (start 94.615 57.15) (end 97.79 60.325) (width 0.5) (layer F.Cu) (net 21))
 (segment (start 101.6 62.23) (end 101.6 63.5) (width 0.5) (layer F.Cu) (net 21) (status 20))
 (segment (start 94.615 55.45) (end 94.615 57.15) (width 0.5) (layer F.Cu) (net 21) (status 10))
 (segment (start 95.885 55.45) (end 95.885 57.15) (width 0.5) (layer F.Cu) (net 22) (status 10))
 (segment (start 95.885 57.15) (end 97.79 59.055) (width 0.5) (layer F.Cu) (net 22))
 (segment (start 97.79 59.055) (end 100.965 59.055) (width 0.5) (layer F.Cu) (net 22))
 (segment (start 104.14 62.23) (end 104.14 63.5) (width 0.5) (layer F.Cu) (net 22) (status 20))
 (segment (start 100.965 59.055) (end 104.14 62.23) (width 0.5) (layer F.Cu) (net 22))
 (segment (start 97.155 57.15) (end 97.155 55.45) (width 0.5) (layer F.Cu) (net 23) (status 20))
 (segment (start 97.79 57.785) (end 97.155 57.15) (width 0.5) (layer F.Cu) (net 23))
 (segment (start 102.87 57.785) (end 97.79 57.785) (width 0.5) (layer F.Cu) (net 23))
 (segment (start 106.68 61.595) (end 102.87 57.785) (width 0.5) (layer F.Cu) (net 23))
 (segment (start 106.68 63.5) (end 106.68 61.595) (width 0.5) (layer F.Cu) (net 23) (status 10))
 (segment (start 118.745 50.165) (end 120.65 48.26) (width 0.5) (layer F.Cu) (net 24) (status 20))
 (segment (start 118.745 52.07) (end 118.745 50.165) (width 0.5) (layer F.Cu) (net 24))
 (segment (start 115.57 55.245) (end 118.745 52.07) (width 0.5) (layer F.Cu) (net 24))
 (segment (start 113.03 55.245) (end 115.57 55.245) (width 0.5) (layer F.Cu) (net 24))
 (segment (start 113.03 53.275) (end 113.03 55.245) (width 0.5) (layer F.Cu) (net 24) (status 10))
 (segment (start 121.92 61.595) (end 121.92 63.5) (width 0.5) (layer F.Cu) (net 5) (status 20))
 (segment (start 121.285 60.96) (end 121.92 61.595) (width 0.5) (layer F.Cu) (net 5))
 (segment (start 120.015 60.96) (end 121.285 60.96) (width 0.5) (layer F.Cu) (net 5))
 (segment (start 118.84 59.785) (end 120.015 60.96) (width 0.5) (layer F.Cu) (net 5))
 (segment (start 118.84 58.42) (end 118.84 59.785) (width 0.5) (layer F.Cu) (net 5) (status 10))
 (segment (start 118.84 57.245) (end 118.84 58.42) (width 0.5) (layer F.Cu) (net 5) (status 20))
 (segment (start 118.11 56.515) (end 118.84 57.245) (width 0.5) (layer F.Cu) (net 5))
 (segment (start 112.395 56.515) (end 118.11 56.515) (width 0.5) (layer F.Cu) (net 5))
 (segment (start 111.76 55.88) (end 112.395 56.515) (width 0.5) (layer F.Cu) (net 5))
 (segment (start 111.76 53.275) (end 111.76 55.88) (width 0.5) (layer F.Cu) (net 5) (status 10))
 (segment (start 119.38 64.77) (end 119.38 63.5) (width 0.5) (layer F.Cu) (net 4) (status 20))
 (segment (start 120.015 65.405) (end 119.38 64.77) (width 0.5) (layer F.Cu) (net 4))
 (segment (start 123.19 65.405) (end 120.015 65.405) (width 0.5) (layer F.Cu) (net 4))
 (segment (start 123.5075 65.0875) (end 123.19 65.405) (width 0.5) (layer F.Cu) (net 4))
 (segment (start 113.03 48.325) (end 114.3 48.325) (width 0.5) (layer F.Cu) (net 4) (status 30))
 (via (at 103.505 42.545) (size 1.5) (drill 0.5) (layers F.Cu B.Cu) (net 4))
 (segment (start 123.46 58.4675) (end 123.5075 58.42) (width 0.5) (layer F.Cu) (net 4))
 (segment (start 121.285 58.4675) (end 123.46 58.4675) (width 0.5) (layer F.Cu) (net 4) (status 10))
 (segment (start 123.5075 58.42) (end 123.5075 65.0875) (width 0.5) (layer F.Cu) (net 4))
 (segment (start 114.3 42.545) (end 106.045 42.545) (width 0.5) (layer F.Cu) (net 4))
 (segment (start 115.57 42.545) (end 114.3 42.545) (width 0.5) (layer F.Cu) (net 4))
 (segment (start 117.475 40.64) (end 115.57 42.545) (width 0.5) (layer F.Cu) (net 4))
 (segment (start 122.555 40.64) (end 117.475 40.64) (width 0.5) (layer F.Cu) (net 4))
 (segment (start 123.5075 41.5925) (end 122.555 40.64) (width 0.5) (layer F.Cu) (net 4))
 (segment (start 106.045 42.545) (end 103.505 42.545) (width 0.5) (layer F.Cu) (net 4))
 (segment (start 114.3 48.325) (end 114.3 46.0375) (width 0.5) (layer F.Cu) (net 4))
 (segment (start 114.3 46.0375) (end 114.935 45.4025) (width 0.5) (layer F.Cu) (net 4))
 (segment (start 114.935 45.4025) (end 123.5075 45.4025) (width 0.5) (layer F.Cu) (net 4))
 (segment (start 123.5075 45.4025) (end 123.5075 41.5925) (width 0.5) (layer F.Cu) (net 4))
 (segment (start 123.5075 58.42) (end 123.5075 45.4025) (width 0.5) (layer F.Cu) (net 4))
 (via (at 100.0125 45.4025) (size 1.5) (drill 0.5) (layers F.Cu B.Cu) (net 4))
 (segment (start 100.0125 45.4025) (end 100.0125 46.0375) (width 0.5) (layer F.Cu) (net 4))
 (segment (start 99.9 46.15) (end 98.425 46.15) (width 0.5) (layer F.Cu) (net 4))
 (segment (start 100.0125 46.0375) (end 99.9 46.15) (width 0.5) (layer F.Cu) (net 4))
 (segment (start 103.505 42.545) (end 102.235 43.815) (width 0.5) (layer B.Cu) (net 4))
 (segment (start 101.6 43.815) (end 100.0125 45.4025) (width 0.5) (layer B.Cu) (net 4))
 (segment (start 102.235 43.815) (end 101.6 43.815) (width 0.5) (layer B.Cu) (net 4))
 (segment (start 111.76 64.77) (end 111.76 63.5) (width 0.5) (layer F.Cu) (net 1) (status 20))
 (segment (start 111.125 65.405) (end 111.76 64.77) (width 0.5) (layer F.Cu) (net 1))
 (segment (start 87.63 65.405) (end 111.125 65.405) (width 0.5) (layer F.Cu) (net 1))
 (segment (start 86.995 64.77) (end 87.63 65.405) (width 0.5) (layer F.Cu) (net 1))
 (segment (start 86.995 55.45) (end 86.995 64.77) (width 0.5) (layer F.Cu) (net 1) (status 10))
 (segment (start 110.49 48.325) (end 111.76 48.325) (width 0.5) (layer F.Cu) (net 25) (status 30))
 (segment (start 88.265 46.15) (end 88.265 44.1325) (width 0.5) (layer F.Cu) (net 26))
 (segment (start 88.265 44.1325) (end 88.5825 43.815) (width 0.5) (layer F.Cu) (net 26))
 (segment (start 88.5825 43.815) (end 100.965 43.815) (width 0.5) (layer F.Cu) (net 26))
 (segment (start 100.965 43.815) (end 101.6 44.45) (width 0.5) (layer F.Cu) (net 26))
 (segment (start 101.6 44.45) (end 101.6 46.99) (width 0.5) (layer F.Cu) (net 26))
 (segment (start 101.6 46.99) (end 101.6 48.26) (width 0.5) (layer F.Cu) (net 26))
 (segment (start 101.6 48.26) (end 100.6475 49.2125) (width 0.5) (layer F.Cu) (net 26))
 (segment (start 100.6475 49.2125) (end 100.33 49.2125) (width 0.5) (layer F.Cu) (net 26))
 (segment (start 106.68 53.275) (end 104.5225 53.275) (width 0.5) (layer F.Cu) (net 26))
 (segment (start 104.5225 53.275) (end 104.14 53.6575) (width 0.5) (layer F.Cu) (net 26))
 (segment (start 104.14 53.6575) (end 104.14 53.6575) (width 0.5) (layer F.Cu) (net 26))
 (via (at 104.14 53.6575) (size 1.5) (drill 0.5) (layers F.Cu B.Cu) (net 26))
 (segment (start 100.33 49.2125) (end 100.33 49.2125) (width 0.5) (layer F.Cu) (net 26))
 (via (at 100.33 49.2125) (size 1.5) (drill 0.5) (layers F.Cu B.Cu) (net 26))
 (segment (start 100.33 49.2125) (end 102.235 51.1175) (width 0.5) (layer B.Cu) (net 26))
 (segment (start 102.235 51.7525) (end 104.14 53.6575) (width 0.5) (layer B.Cu) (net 26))
 (segment (start 102.235 51.1175) (end 102.235 51.7525) (width 0.5) (layer B.Cu) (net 26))
 (segment (start 107.95 53.275) (end 110.49 53.275) (width 0.5) (layer F.Cu) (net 27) (status 30)))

